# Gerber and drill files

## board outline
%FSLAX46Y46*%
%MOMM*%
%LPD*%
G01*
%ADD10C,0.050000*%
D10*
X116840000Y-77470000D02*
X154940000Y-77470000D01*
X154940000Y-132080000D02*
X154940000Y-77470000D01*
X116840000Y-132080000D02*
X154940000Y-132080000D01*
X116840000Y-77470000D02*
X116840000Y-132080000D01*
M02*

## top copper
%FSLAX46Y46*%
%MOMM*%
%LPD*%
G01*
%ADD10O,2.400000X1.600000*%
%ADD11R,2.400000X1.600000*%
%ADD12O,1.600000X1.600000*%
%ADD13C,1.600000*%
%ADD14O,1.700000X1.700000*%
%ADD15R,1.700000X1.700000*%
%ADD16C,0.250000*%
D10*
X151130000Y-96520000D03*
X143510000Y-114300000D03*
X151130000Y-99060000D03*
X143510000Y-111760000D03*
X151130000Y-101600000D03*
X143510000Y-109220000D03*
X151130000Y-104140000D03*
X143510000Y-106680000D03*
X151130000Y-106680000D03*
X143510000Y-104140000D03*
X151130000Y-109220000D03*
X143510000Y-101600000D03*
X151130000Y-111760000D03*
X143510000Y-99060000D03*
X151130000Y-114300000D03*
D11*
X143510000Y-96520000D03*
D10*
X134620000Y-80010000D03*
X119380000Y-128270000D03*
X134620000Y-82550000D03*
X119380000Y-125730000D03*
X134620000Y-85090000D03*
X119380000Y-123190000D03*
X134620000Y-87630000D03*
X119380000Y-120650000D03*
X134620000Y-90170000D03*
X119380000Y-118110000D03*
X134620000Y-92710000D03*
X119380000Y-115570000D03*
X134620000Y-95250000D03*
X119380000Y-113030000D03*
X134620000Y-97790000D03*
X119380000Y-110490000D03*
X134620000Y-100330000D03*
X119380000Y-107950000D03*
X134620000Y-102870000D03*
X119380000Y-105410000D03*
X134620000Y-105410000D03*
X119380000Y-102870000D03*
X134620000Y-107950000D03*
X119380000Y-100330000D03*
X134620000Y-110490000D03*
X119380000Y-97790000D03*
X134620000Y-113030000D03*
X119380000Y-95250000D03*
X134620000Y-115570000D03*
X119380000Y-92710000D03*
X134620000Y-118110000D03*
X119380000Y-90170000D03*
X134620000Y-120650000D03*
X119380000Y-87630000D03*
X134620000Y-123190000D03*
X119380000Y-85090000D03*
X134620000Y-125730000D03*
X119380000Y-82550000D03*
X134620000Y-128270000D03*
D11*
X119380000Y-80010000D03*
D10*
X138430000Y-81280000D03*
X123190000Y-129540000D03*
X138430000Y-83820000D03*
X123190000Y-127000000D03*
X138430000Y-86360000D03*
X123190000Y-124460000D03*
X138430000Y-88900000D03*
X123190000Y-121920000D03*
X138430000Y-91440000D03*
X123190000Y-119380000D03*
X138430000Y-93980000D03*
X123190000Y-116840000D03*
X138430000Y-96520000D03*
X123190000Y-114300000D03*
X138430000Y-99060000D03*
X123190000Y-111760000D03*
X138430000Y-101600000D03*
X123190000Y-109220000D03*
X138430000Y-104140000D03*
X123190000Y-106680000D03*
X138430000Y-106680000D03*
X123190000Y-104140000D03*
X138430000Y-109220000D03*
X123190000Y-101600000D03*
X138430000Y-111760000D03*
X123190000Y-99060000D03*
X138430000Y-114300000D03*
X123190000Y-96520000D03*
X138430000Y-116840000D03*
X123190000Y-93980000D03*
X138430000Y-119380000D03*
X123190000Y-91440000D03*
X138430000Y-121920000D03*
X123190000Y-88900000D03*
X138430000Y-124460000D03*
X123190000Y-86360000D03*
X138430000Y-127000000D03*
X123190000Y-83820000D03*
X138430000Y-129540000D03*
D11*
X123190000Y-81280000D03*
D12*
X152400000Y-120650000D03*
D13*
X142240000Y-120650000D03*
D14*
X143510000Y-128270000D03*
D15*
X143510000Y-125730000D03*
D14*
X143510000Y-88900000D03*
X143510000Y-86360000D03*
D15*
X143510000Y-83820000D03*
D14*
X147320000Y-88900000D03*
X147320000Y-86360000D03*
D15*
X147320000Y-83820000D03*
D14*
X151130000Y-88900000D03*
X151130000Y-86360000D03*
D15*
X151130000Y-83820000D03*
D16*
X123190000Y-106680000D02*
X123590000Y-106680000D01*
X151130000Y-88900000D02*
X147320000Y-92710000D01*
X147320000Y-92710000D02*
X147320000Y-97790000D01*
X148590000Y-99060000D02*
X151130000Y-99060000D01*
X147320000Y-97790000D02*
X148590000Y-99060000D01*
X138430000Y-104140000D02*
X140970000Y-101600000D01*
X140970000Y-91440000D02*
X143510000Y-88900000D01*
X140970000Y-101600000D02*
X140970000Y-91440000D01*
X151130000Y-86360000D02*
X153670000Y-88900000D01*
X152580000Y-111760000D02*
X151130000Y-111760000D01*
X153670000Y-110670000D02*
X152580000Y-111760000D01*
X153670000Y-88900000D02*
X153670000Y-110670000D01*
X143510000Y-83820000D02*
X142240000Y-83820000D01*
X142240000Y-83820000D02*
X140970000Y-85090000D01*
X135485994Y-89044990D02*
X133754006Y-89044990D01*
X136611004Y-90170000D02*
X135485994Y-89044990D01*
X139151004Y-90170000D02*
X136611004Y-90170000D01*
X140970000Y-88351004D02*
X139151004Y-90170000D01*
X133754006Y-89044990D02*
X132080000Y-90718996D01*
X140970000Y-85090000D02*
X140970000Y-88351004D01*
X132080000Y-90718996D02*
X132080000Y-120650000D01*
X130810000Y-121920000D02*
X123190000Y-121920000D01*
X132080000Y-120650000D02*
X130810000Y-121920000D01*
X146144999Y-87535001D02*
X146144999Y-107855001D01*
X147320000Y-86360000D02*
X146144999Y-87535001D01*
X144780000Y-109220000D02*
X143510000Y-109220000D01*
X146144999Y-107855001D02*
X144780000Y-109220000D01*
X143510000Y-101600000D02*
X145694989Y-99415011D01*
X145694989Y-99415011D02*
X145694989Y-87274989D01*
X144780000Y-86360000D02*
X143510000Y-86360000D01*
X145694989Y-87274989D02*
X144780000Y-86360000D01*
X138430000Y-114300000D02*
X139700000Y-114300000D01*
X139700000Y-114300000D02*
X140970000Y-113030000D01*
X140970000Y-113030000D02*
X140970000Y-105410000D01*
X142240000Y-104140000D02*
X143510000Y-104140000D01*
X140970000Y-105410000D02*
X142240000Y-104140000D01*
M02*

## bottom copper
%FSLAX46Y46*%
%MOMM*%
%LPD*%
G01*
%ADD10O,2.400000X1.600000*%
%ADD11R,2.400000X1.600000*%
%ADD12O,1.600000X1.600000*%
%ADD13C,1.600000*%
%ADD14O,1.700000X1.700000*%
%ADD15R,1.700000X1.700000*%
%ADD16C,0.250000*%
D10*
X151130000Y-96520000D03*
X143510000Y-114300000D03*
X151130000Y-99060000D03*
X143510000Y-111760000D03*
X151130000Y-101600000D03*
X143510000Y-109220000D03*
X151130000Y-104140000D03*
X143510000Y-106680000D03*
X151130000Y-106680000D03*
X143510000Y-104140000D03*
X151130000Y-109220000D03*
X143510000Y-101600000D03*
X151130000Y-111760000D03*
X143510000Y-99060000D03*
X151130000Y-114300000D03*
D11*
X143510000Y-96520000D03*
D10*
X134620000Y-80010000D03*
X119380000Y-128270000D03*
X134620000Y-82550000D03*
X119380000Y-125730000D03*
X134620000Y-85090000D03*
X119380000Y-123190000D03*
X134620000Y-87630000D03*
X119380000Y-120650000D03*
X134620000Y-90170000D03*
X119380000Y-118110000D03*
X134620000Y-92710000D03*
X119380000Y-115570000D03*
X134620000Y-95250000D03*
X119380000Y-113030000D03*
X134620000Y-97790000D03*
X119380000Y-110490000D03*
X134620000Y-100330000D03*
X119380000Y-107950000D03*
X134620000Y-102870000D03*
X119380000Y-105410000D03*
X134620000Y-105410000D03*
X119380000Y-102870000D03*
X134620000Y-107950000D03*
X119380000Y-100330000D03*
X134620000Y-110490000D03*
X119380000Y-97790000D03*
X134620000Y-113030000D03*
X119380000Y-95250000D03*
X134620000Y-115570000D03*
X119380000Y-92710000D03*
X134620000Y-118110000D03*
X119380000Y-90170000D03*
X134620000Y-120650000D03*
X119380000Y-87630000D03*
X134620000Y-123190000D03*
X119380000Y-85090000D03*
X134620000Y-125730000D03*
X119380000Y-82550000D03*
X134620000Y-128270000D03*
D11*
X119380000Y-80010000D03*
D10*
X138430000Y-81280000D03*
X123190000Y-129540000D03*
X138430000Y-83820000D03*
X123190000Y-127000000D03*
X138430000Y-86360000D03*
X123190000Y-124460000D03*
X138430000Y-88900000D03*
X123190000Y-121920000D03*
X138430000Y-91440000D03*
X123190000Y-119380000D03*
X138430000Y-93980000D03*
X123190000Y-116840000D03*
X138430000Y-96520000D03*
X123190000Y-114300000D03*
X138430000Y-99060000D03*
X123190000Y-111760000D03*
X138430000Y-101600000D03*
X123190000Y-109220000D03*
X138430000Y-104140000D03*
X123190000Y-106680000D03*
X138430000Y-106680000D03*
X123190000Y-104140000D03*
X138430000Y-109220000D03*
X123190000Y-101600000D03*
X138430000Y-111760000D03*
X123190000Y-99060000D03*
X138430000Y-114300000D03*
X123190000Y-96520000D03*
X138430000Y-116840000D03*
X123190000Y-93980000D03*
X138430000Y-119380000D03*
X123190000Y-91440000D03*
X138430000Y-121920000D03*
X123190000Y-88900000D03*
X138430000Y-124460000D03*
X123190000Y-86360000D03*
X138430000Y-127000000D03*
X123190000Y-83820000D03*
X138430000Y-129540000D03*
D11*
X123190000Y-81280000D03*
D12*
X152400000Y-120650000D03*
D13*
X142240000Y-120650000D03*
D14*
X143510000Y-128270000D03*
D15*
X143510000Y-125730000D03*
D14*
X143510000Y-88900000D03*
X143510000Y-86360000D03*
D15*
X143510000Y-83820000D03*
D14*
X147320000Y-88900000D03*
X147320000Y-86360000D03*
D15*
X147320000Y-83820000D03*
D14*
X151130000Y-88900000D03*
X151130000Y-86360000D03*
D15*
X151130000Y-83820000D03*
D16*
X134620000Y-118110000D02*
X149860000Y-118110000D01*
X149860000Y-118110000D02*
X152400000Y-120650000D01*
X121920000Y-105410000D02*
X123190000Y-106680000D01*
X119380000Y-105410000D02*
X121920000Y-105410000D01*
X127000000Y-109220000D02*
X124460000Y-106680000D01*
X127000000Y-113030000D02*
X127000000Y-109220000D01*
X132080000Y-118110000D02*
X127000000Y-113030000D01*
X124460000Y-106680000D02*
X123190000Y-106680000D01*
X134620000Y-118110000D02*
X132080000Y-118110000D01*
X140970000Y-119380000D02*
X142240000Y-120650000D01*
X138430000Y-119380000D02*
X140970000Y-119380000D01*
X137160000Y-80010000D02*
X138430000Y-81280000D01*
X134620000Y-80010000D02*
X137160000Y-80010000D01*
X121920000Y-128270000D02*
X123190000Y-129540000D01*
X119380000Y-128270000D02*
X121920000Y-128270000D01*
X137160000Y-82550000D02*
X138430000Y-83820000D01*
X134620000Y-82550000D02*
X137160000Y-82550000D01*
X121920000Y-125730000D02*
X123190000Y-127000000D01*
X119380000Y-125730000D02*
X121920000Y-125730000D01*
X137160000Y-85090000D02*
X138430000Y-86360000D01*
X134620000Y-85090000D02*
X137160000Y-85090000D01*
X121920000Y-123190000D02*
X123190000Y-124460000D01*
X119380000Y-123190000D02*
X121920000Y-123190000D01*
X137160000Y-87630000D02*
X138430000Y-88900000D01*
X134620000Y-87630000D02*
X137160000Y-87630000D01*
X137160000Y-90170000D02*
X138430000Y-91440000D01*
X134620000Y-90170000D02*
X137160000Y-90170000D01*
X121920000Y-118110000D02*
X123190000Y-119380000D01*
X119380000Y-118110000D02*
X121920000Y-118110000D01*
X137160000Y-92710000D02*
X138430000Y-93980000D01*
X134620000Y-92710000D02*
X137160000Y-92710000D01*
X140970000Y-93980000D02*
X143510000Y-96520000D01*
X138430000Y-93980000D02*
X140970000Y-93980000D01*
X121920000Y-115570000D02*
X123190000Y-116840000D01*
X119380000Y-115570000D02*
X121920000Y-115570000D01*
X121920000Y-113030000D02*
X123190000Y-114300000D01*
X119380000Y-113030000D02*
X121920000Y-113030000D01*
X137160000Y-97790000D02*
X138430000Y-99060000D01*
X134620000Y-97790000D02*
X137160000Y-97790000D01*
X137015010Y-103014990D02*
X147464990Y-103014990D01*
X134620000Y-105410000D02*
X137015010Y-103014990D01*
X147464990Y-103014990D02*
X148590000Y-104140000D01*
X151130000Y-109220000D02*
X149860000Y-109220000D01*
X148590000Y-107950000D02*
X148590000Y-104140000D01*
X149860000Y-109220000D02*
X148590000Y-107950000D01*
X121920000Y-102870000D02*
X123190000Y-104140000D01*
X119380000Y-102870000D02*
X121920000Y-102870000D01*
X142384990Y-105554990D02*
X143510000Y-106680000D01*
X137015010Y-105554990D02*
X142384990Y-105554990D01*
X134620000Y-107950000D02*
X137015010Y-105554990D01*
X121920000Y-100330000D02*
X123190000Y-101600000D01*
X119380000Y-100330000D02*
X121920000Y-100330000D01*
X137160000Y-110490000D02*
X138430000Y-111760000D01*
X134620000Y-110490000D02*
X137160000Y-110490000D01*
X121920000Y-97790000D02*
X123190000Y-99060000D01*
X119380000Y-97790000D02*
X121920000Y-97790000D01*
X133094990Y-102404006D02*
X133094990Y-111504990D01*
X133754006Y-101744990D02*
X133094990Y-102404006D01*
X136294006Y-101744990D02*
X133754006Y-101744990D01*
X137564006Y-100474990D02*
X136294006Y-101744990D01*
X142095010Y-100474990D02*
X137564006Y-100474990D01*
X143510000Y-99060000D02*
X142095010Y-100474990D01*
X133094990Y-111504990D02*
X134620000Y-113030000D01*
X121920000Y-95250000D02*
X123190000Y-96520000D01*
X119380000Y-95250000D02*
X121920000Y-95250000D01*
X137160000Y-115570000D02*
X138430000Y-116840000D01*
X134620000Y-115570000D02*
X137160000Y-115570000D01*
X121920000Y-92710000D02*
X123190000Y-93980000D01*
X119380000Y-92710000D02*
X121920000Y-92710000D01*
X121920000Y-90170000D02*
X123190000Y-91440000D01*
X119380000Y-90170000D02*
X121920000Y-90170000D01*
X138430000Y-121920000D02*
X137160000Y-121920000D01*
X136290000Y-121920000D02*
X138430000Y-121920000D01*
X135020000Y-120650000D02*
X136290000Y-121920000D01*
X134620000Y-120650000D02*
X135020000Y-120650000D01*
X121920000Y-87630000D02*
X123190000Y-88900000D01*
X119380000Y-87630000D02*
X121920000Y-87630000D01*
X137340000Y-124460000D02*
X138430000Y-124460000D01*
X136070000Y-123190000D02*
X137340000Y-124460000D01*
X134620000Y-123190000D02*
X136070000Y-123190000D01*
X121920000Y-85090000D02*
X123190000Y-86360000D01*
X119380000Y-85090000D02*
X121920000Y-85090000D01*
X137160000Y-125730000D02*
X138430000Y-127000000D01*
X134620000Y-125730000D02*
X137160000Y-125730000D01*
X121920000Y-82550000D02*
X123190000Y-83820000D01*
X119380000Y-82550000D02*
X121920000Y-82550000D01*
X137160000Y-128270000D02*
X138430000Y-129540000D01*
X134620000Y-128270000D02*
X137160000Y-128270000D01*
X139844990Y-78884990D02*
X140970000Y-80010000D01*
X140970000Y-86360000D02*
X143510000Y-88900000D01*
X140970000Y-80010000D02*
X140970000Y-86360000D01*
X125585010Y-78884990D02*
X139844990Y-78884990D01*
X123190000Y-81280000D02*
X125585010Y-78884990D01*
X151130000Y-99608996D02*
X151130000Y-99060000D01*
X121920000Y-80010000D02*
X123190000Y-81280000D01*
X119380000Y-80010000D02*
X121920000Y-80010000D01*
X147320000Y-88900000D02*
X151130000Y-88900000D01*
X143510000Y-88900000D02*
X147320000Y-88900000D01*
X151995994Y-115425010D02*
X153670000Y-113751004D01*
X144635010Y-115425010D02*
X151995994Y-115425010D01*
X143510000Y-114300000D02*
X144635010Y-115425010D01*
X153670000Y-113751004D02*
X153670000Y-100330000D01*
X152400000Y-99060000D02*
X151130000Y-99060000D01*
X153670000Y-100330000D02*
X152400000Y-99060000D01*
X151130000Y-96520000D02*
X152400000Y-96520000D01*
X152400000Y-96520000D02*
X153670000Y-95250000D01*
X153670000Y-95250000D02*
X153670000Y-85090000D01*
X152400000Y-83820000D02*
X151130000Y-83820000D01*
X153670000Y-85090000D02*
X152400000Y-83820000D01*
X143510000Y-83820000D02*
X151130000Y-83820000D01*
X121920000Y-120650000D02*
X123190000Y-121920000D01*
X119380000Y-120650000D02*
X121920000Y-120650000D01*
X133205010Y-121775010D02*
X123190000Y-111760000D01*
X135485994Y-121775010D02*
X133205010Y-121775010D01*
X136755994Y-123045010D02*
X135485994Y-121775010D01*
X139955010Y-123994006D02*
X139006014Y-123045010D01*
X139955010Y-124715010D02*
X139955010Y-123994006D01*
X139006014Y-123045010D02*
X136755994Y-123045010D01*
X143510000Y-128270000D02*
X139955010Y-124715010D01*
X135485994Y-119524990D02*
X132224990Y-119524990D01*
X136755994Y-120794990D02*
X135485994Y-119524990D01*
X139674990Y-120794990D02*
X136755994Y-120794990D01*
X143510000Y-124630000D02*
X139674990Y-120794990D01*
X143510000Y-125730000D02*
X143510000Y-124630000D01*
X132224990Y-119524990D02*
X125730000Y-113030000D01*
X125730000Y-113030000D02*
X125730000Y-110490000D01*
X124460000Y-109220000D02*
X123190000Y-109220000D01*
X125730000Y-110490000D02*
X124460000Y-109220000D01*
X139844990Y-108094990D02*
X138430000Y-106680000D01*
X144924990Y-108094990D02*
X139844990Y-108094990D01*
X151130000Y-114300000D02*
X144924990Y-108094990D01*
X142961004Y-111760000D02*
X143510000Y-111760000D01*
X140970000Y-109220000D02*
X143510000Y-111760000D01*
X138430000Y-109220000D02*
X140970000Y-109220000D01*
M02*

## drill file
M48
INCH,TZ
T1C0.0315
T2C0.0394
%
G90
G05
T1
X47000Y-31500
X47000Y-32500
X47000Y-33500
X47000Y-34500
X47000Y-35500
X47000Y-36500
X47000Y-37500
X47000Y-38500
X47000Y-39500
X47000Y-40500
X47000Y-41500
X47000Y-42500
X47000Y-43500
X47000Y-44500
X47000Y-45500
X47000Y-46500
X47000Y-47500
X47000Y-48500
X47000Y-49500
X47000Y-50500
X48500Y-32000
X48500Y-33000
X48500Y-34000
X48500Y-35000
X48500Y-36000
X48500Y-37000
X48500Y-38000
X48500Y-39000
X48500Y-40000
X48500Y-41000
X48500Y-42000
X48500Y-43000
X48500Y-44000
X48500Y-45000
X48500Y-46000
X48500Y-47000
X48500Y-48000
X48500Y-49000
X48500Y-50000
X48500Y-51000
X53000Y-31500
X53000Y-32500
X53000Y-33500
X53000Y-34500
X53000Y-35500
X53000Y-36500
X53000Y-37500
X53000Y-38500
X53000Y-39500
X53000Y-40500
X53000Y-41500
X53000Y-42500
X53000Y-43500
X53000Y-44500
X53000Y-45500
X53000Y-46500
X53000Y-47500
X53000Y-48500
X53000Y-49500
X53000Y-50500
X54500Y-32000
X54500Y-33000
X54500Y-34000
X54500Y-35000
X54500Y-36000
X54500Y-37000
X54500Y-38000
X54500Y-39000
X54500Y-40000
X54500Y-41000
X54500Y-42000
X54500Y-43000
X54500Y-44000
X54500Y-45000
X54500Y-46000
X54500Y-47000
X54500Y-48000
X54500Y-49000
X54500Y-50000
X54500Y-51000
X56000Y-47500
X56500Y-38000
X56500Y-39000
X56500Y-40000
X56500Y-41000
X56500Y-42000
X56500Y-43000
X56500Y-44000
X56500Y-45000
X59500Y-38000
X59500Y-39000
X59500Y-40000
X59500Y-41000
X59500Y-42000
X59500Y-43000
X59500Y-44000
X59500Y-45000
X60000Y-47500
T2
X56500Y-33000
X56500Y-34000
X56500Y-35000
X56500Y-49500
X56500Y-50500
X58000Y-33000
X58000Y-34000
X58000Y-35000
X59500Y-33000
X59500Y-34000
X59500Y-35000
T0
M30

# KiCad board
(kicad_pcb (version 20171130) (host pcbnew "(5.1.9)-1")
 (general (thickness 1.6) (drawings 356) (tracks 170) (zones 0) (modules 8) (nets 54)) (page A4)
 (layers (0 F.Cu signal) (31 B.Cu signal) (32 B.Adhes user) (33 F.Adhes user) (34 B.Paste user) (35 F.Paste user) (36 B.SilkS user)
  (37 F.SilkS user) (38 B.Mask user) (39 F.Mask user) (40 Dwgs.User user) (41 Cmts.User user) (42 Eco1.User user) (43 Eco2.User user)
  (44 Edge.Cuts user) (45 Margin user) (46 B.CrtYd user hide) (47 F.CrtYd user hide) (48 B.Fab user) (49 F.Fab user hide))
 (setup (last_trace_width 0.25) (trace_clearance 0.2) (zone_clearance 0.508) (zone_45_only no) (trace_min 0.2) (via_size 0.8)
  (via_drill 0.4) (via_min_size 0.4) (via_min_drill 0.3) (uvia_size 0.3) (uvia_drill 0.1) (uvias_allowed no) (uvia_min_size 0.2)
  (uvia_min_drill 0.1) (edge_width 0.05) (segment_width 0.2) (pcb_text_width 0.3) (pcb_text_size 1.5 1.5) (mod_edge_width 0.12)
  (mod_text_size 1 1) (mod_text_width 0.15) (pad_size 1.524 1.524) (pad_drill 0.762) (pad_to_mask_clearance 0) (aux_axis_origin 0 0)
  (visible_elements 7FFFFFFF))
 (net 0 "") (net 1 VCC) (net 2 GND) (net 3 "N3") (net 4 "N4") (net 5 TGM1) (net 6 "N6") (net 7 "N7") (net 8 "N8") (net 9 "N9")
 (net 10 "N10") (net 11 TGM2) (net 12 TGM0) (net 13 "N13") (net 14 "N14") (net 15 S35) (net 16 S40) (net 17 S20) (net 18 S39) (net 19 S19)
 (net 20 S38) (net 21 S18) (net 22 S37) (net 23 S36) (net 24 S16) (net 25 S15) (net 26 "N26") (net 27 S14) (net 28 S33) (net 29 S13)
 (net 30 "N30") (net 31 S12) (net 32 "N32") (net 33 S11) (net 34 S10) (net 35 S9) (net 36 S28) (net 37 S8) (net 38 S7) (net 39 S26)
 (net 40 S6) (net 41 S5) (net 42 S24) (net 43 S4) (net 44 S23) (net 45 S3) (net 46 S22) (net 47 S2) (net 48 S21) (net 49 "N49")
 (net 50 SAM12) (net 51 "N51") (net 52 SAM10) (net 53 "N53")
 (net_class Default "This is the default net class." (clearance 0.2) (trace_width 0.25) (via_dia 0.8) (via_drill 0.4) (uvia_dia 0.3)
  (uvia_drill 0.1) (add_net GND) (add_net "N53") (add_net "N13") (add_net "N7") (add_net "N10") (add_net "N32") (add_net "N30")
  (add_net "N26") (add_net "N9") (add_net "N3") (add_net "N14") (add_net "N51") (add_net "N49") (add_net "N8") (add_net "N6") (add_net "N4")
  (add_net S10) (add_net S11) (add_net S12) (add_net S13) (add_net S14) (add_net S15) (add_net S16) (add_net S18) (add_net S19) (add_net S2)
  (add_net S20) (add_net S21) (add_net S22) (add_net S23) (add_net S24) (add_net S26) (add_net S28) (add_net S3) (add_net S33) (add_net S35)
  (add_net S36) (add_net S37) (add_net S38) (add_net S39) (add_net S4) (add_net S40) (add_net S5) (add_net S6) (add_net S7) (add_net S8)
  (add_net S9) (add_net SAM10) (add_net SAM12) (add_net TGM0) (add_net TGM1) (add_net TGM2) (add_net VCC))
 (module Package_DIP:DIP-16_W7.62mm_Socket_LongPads (layer F.Cu) (at 143.51 96.52)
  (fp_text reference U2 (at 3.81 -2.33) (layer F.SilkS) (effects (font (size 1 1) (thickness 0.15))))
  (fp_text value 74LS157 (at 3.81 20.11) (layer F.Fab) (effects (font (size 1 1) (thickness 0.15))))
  (pad 16 thru_hole oval (at 7.62 0) (size 2.4 1.6) (drill 0.8) (layers *.Cu *.Mask) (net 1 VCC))
  (pad 8 thru_hole oval (at 0 17.78) (size 2.4 1.6) (drill 0.8) (layers *.Cu *.Mask) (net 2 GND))
  (pad 15 thru_hole oval (at 7.62 2.54) (size 2.4 1.6) (drill 0.8) (layers *.Cu *.Mask) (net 2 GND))
  (pad 7 thru_hole oval (at 0 15.24) (size 2.4 1.6) (drill 0.8) (layers *.Cu *.Mask) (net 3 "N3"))
  (pad 14 thru_hole oval (at 7.62 5.08) (size 2.4 1.6) (drill 0.8) (layers *.Cu *.Mask) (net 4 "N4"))
  (pad 6 thru_hole oval (at 0 12.7) (size 2.4 1.6) (drill 0.8) (layers *.Cu *.Mask) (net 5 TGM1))
  (pad 13 thru_hole oval (at 7.62 7.62) (size 2.4 1.6) (drill 0.8) (layers *.Cu *.Mask) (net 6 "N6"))
  (pad 5 thru_hole oval (at 0 10.16) (size 2.4 1.6) (drill 0.8) (layers *.Cu *.Mask) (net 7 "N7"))
  (pad 12 thru_hole oval (at 7.62 10.16) (size 2.4 1.6) (drill 0.8) (layers *.Cu *.Mask) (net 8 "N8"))
  (pad 4 thru_hole oval (at 0 7.62) (size 2.4 1.6) (drill 0.8) (layers *.Cu *.Mask) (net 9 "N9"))
  (pad 11 thru_hole oval (at 7.62 12.7) (size 2.4 1.6) (drill 0.8) (layers *.Cu *.Mask) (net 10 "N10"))
  (pad 3 thru_hole oval (at 0 5.08) (size 2.4 1.6) (drill 0.8) (layers *.Cu *.Mask) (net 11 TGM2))
  (pad 10 thru_hole oval (at 7.62 15.24) (size 2.4 1.6) (drill 0.8) (layers *.Cu *.Mask) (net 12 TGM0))
  (pad 2 thru_hole oval (at 0 2.54) (size 2.4 1.6) (drill 0.8) (layers *.Cu *.Mask) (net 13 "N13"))
  (pad 9 thru_hole oval (at 7.62 17.78) (size 2.4 1.6) (drill 0.8) (layers *.Cu *.Mask) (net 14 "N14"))
  (pad 1 thru_hole rect (at 0 0) (size 2.4 1.6) (drill 0.8) (layers *.Cu *.Mask) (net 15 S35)))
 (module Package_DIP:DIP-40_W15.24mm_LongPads (layer F.Cu) (at 119.38 80.01)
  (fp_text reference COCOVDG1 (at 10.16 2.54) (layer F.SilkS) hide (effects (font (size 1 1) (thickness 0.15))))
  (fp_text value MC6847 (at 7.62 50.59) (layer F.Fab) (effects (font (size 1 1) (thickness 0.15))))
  (pad 40 thru_hole oval (at 15.24 0) (size 2.4 1.6) (drill 0.8) (layers *.Cu *.Mask) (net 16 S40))
  (pad 20 thru_hole oval (at 0 48.26) (size 2.4 1.6) (drill 0.8) (layers *.Cu *.Mask) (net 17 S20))
  (pad 39 thru_hole oval (at 15.24 2.54) (size 2.4 1.6) (drill 0.8) (layers *.Cu *.Mask) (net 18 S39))
  (pad 19 thru_hole oval (at 0 45.72) (size 2.4 1.6) (drill 0.8) (layers *.Cu *.Mask) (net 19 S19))
  (pad 38 thru_hole oval (at 15.24 5.08) (size 2.4 1.6) (drill 0.8) (layers *.Cu *.Mask) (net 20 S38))
  (pad 18 thru_hole oval (at 0 43.18) (size 2.4 1.6) (drill 0.8) (layers *.Cu *.Mask) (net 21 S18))
  (pad 37 thru_hole oval (at 15.24 7.62) (size 2.4 1.6) (drill 0.8) (layers *.Cu *.Mask) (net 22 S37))
  (pad 17 thru_hole oval (at 0 40.64) (size 2.4 1.6) (drill 0.8) (layers *.Cu *.Mask) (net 1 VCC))
  (pad 36 thru_hole oval (at 15.24 10.16) (size 2.4 1.6) (drill 0.8) (layers *.Cu *.Mask) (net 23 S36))
  (pad 16 thru_hole oval (at 0 38.1) (size 2.4 1.6) (drill 0.8) (layers *.Cu *.Mask) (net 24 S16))
  (pad 35 thru_hole oval (at 15.24 12.7) (size 2.4 1.6) (drill 0.8) (layers *.Cu *.Mask) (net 15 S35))
  (pad 15 thru_hole oval (at 0 35.56) (size 2.4 1.6) (drill 0.8) (layers *.Cu *.Mask) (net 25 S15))
  (pad 34 thru_hole oval (at 15.24 15.24) (size 2.4 1.6) (drill 0.8) (layers *.Cu *.Mask) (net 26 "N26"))
  (pad 14 thru_hole oval (at 0 33.02) (size 2.4 1.6) (drill 0.8) (layers *.Cu *.Mask) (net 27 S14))
  (pad 33 thru_hole oval (at 15.24 17.78) (size 2.4 1.6) (drill 0.8) (layers *.Cu *.Mask) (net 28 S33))
  (pad 13 thru_hole oval (at 0 30.48) (size 2.4 1.6) (drill 0.8) (layers *.Cu *.Mask) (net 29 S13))
  (pad 32 thru_hole oval (at 15.24 20.32) (size 2.4 1.6) (drill 0.8) (layers *.Cu *.Mask) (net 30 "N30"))
  (pad 12 thru_hole oval (at 0 27.94) (size 2.4 1.6) (drill 0.8) (layers *.Cu *.Mask) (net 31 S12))
  (pad 31 thru_hole oval (at 15.24 22.86) (size 2.4 1.6) (drill 0.8) (layers *.Cu *.Mask) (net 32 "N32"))
  (pad 11 thru_hole oval (at 0 25.4) (size 2.4 1.6) (drill 0.8) (layers *.Cu *.Mask) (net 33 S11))
  (pad 30 thru_hole oval (at 15.24 25.4) (size 2.4 1.6) (drill 0.8) (layers *.Cu *.Mask) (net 10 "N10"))
  (pad 10 thru_hole oval (at 0 22.86) (size 2.4 1.6) (drill 0.8) (layers *.Cu *.Mask) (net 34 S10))
  (pad 29 thru_hole oval (at 15.24 27.94) (size 2.4 1.6) (drill 0.8) (layers *.Cu *.Mask) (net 7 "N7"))
  (pad 9 thru_hole oval (at 0 20.32) (size 2.4 1.6) (drill 0.8) (layers *.Cu *.Mask) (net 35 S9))
  (pad 28 thru_hole oval (at 15.24 30.48) (size 2.4 1.6) (drill 0.8) (layers *.Cu *.Mask) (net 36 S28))
  (pad 8 thru_hole oval (at 0 17.78) (size 2.4 1.6) (drill 0.8) (layers *.Cu *.Mask) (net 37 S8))
  (pad 27 thru_hole oval (at 15.24 33.02) (size 2.4 1.6) (drill 0.8) (layers *.Cu *.Mask) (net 13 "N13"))
  (pad 7 thru_hole oval (at 0 15.24) (size 2.4 1.6) (drill 0.8) (layers *.Cu *.Mask) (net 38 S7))
  (pad 26 thru_hole oval (at 15.24 35.56) (size 2.4 1.6) (drill 0.8) (layers *.Cu *.Mask) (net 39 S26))
  (pad 6 thru_hole oval (at 0 12.7) (size 2.4 1.6) (drill 0.8) (layers *.Cu *.Mask) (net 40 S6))
  (pad 25 thru_hole oval (at 15.24 38.1) (size 2.4 1.6) (drill 0.8) (layers *.Cu *.Mask) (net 33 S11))
  (pad 5 thru_hole oval (at 0 10.16) (size 2.4 1.6) (drill 0.8) (layers *.Cu *.Mask) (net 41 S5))
  (pad 24 thru_hole oval (at 15.24 40.64) (size 2.4 1.6) (drill 0.8) (layers *.Cu *.Mask) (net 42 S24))
  (pad 4 thru_hole oval (at 0 7.62) (size 2.4 1.6) (drill 0.8) (layers *.Cu *.Mask) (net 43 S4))
  (pad 23 thru_hole oval (at 15.24 43.18) (size 2.4 1.6) (drill 0.8) (layers *.Cu *.Mask) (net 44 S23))
  (pad 3 thru_hole oval (at 0 5.08) (size 2.4 1.6) (drill 0.8) (layers *.Cu *.Mask) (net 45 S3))
  (pad 22 thru_hole oval (at 15.24 45.72) (size 2.4 1.6) (drill 0.8) (layers *.Cu *.Mask) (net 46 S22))
  (pad 2 thru_hole oval (at 0 2.54) (size 2.4 1.6) (drill 0.8) (layers *.Cu *.Mask) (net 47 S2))
  (pad 21 thru_hole oval (at 15.24 48.26) (size 2.4 1.6) (drill 0.8) (layers *.Cu *.Mask) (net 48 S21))
  (pad 1 thru_hole rect (at 0 0) (size 2.4 1.6) (drill 0.8) (layers *.Cu *.Mask) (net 2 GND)))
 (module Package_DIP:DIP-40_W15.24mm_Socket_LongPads (layer F.Cu) (at 123.19 81.28)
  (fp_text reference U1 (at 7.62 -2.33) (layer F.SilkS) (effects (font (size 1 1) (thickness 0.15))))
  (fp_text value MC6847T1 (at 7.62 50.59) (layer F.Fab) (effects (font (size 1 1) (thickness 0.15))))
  (pad 40 thru_hole oval (at 15.24 0) (size 2.4 1.6) (drill 0.8) (layers *.Cu *.Mask) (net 16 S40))
  (pad 20 thru_hole oval (at 0 48.26) (size 2.4 1.6) (drill 0.8) (layers *.Cu *.Mask) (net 17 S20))
  (pad 39 thru_hole oval (at 15.24 2.54) (size 2.4 1.6) (drill 0.8) (layers *.Cu *.Mask) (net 18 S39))
  (pad 19 thru_hole oval (at 0 45.72) (size 2.4 1.6) (drill 0.8) (layers *.Cu *.Mask) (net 19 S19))
  (pad 38 thru_hole oval (at 15.24 5.08) (size 2.4 1.6) (drill 0.8) (layers *.Cu *.Mask) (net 20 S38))
  (pad 18 thru_hole oval (at 0 43.18) (size 2.4 1.6) (drill 0.8) (layers *.Cu *.Mask) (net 21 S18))
  (pad 37 thru_hole oval (at 15.24 7.62) (size 2.4 1.6) (drill 0.8) (layers *.Cu *.Mask) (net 22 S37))
  (pad 17 thru_hole oval (at 0 40.64) (size 2.4 1.6) (drill 0.8) (layers *.Cu *.Mask) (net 1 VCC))
  (pad 36 thru_hole oval (at 15.24 10.16) (size 2.4 1.6) (drill 0.8) (layers *.Cu *.Mask) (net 23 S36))
  (pad 16 thru_hole oval (at 0 38.1) (size 2.4 1.6) (drill 0.8) (layers *.Cu *.Mask) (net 24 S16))
  (pad 35 thru_hole oval (at 15.24 12.7) (size 2.4 1.6) (drill 0.8) (layers *.Cu *.Mask) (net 15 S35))
  (pad 15 thru_hole oval (at 0 35.56) (size 2.4 1.6) (drill 0.8) (layers *.Cu *.Mask) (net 25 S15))
  (pad 34 thru_hole oval (at 15.24 15.24) (size 2.4 1.6) (drill 0.8) (layers *.Cu *.Mask) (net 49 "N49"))
  (pad 14 thru_hole oval (at 0 33.02) (size 2.4 1.6) (drill 0.8) (layers *.Cu *.Mask) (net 27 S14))
  (pad 33 thru_hole oval (at 15.24 17.78) (size 2.4 1.6) (drill 0.8) (layers *.Cu *.Mask) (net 28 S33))
  (pad 13 thru_hole oval (at 0 30.48) (size 2.4 1.6) (drill 0.8) (layers *.Cu *.Mask) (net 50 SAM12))
  (pad 32 thru_hole oval (at 15.24 20.32) (size 2.4 1.6) (drill 0.8) (layers *.Cu *.Mask) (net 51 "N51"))
  (pad 12 thru_hole oval (at 0 27.94) (size 2.4 1.6) (drill 0.8) (layers *.Cu *.Mask) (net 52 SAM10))
  (pad 31 thru_hole oval (at 15.24 22.86) (size 2.4 1.6) (drill 0.8) (layers *.Cu *.Mask) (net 2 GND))
  (pad 11 thru_hole oval (at 0 25.4) (size 2.4 1.6) (drill 0.8) (layers *.Cu *.Mask) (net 33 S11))
  (pad 30 thru_hole oval (at 15.24 25.4) (size 2.4 1.6) (drill 0.8) (layers *.Cu *.Mask) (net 14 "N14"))
  (pad 10 thru_hole oval (at 0 22.86) (size 2.4 1.6) (drill 0.8) (layers *.Cu *.Mask) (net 34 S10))
  (pad 29 thru_hole oval (at 15.24 27.94) (size 2.4 1.6) (drill 0.8) (layers *.Cu *.Mask) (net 3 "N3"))
  (pad 9 thru_hole oval (at 0 20.32) (size 2.4 1.6) (drill 0.8) (layers *.Cu *.Mask) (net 35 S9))
  (pad 28 thru_hole oval (at 15.24 30.48) (size 2.4 1.6) (drill 0.8) (layers *.Cu *.Mask) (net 36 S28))
  (pad 8 thru_hole oval (at 0 17.78) (size 2.4 1.6) (drill 0.8) (layers *.Cu *.Mask) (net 37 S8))
  (pad 27 thru_hole oval (at 15.24 33.02) (size 2.4 1.6) (drill 0.8) (layers *.Cu *.Mask) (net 9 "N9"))
  (pad 7 thru_hole oval (at 0 15.24) (size 2.4 1.6) (drill 0.8) (layers *.Cu *.Mask) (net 38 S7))
  (pad 26 thru_hole oval (at 15.24 35.56) (size 2.4 1.6) (drill 0.8) (layers *.Cu *.Mask) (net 39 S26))
  (pad 6 thru_hole oval (at 0 12.7) (size 2.4 1.6) (drill 0.8) (layers *.Cu *.Mask) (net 40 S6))
  (pad 25 thru_hole oval (at 15.24 38.1) (size 2.4 1.6) (drill 0.8) (layers *.Cu *.Mask) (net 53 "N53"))
  (pad 5 thru_hole oval (at 0 10.16) (size 2.4 1.6) (drill 0.8) (layers *.Cu *.Mask) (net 41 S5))
  (pad 24 thru_hole oval (at 15.24 40.64) (size 2.4 1.6) (drill 0.8) (layers *.Cu *.Mask) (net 42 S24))
  (pad 4 thru_hole oval (at 0 7.62) (size 2.4 1.6) (drill 0.8) (layers *.Cu *.Mask) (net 43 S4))
  (pad 23 thru_hole oval (at 15.24 43.18) (size 2.4 1.6) (drill 0.8) (layers *.Cu *.Mask) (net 44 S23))
  (pad 3 thru_hole oval (at 0 5.08) (size 2.4 1.6) (drill 0.8) (layers *.Cu *.Mask) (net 45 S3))
  (pad 22 thru_hole oval (at 15.24 45.72) (size 2.4 1.6) (drill 0.8) (layers *.Cu *.Mask) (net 46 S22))
  (pad 2 thru_hole oval (at 0 2.54) (size 2.4 1.6) (drill 0.8) (layers *.Cu *.Mask) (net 47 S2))
  (pad 21 thru_hole oval (at 15.24 48.26) (size 2.4 1.6) (drill 0.8) (layers *.Cu *.Mask) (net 48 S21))
  (pad 1 thru_hole rect (at 0 0) (size 2.4 1.6) (drill 0.8) (layers *.Cu *.Mask) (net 2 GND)))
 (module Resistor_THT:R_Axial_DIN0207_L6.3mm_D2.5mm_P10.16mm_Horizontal (layer F.Cu) (at 142.24 120.65)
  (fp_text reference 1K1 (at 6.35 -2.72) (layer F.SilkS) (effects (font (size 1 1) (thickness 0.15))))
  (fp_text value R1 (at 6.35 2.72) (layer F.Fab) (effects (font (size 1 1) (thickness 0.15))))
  (pad 2 thru_hole oval (at 10.16 0) (size 1.6 1.6) (drill 0.8) (layers *.Cu *.Mask) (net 33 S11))
  (pad 1 thru_hole circle (at 0 0) (size 1.6 1.6) (drill 0.8) (layers *.Cu *.Mask) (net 53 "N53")))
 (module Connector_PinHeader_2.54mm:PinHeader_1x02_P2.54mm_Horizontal (layer F.Cu) (at 143.51 125.73)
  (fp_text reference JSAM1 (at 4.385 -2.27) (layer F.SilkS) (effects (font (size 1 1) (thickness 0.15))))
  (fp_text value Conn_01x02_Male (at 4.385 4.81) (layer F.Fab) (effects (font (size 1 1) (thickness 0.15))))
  (pad 2 thru_hole oval (at 0 2.54) (size 1.7 1.7) (drill 1) (layers *.Cu *.Mask) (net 50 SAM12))
  (pad 1 thru_hole rect (at 0 0) (size 1.7 1.7) (drill 1) (layers *.Cu *.Mask) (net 52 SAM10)))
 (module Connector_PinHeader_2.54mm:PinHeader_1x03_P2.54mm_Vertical (layer F.Cu) (at 143.51 83.82)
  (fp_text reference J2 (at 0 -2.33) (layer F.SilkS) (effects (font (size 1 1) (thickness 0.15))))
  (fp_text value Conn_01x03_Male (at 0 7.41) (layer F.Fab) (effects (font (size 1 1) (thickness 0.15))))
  (pad 3 thru_hole oval (at 0 5.08) (size 1.7 1.7) (drill 1) (layers *.Cu *.Mask) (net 2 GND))
  (pad 2 thru_hole oval (at 0 2.54) (size 1.7 1.7) (drill 1) (layers *.Cu *.Mask) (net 11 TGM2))
  (pad 1 thru_hole rect (at 0 0) (size 1.7 1.7) (drill 1) (layers *.Cu *.Mask) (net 1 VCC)))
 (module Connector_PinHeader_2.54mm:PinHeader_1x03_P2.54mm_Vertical (layer F.Cu) (at 147.32 83.82)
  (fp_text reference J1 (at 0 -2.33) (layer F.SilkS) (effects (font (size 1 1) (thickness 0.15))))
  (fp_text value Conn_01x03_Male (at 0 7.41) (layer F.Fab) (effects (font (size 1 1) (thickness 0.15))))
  (pad 3 thru_hole oval (at 0 5.08) (size 1.7 1.7) (drill 1) (layers *.Cu *.Mask) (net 2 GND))
  (pad 2 thru_hole oval (at 0 2.54) (size 1.7 1.7) (drill 1) (layers *.Cu *.Mask) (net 5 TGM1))
  (pad 1 thru_hole rect (at 0 0) (size 1.7 1.7) (drill 1) (layers *.Cu *.Mask) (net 1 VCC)))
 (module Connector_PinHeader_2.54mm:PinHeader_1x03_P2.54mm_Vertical (layer F.Cu) (at 151.13 83.82)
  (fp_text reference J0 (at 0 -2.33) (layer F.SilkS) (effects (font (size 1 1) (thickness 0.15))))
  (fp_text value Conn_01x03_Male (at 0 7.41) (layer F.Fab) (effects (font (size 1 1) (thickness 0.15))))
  (pad 3 thru_hole oval (at 0 5.08) (size 1.7 1.7) (drill 1) (layers *.Cu *.Mask) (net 2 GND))
  (pad 2 thru_hole oval (at 0 2.54) (size 1.7 1.7) (drill 1) (layers *.Cu *.Mask) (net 12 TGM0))
  (pad 1 thru_hole rect (at 0 0) (size 1.7 1.7) (drill 1) (layers *.Cu *.Mask) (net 1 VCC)))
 (gr_line (start 116.84 77.47) (end 154.94 77.47) (layer Edge.Cuts) (width 0.05))
 (gr_line (start 154.94 132.08) (end 154.94 77.47) (layer Edge.Cuts) (width 0.05))
 (gr_line (start 116.84 132.08) (end 154.94 132.08) (layer Edge.Cuts) (width 0.05))
 (gr_line (start 116.84 77.47) (end 116.84 132.08) (layer Edge.Cuts) (width 0.05))
 (segment (start 123.19 106.68) (end 123.59 106.68) (width 0.25) (layer F.Cu) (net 33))
 (segment (start 134.62 118.11) (end 149.86 118.11) (width 0.25) (layer B.Cu) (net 33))
 (segment (start 149.86 118.11) (end 152.4 120.65) (width 0.25) (layer B.Cu) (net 33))
 (segment (start 121.92 105.41) (end 123.19 106.68) (width 0.25) (layer B.Cu) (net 33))
 (segment (start 119.38 105.41) (end 121.92 105.41) (width 0.25) (layer B.Cu) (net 33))
 (segment (start 127 109.22) (end 124.46 106.68) (width 0.25) (layer B.Cu) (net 33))
 (segment (start 127 113.03) (end 127 109.22) (width 0.25) (layer B.Cu) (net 33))
 (segment (start 132.08 118.11) (end 127 113.03) (width 0.25) (layer B.Cu) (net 33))
 (segment (start 124.46 106.68) (end 123.19 106.68) (width 0.25) (layer B.Cu) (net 33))
 (segment (start 134.62 118.11) (end 132.08 118.11) (width 0.25) (layer B.Cu) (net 33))
 (segment (start 140.97 119.38) (end 142.24 120.65) (width 0.25) (layer B.Cu) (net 53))
 (segment (start 138.43 119.38) (end 140.97 119.38) (width 0.25) (layer B.Cu) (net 53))
 (segment (start 137.16 80.01) (end 138.43 81.28) (width 0.25) (layer B.Cu) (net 16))
 (segment (start 134.62 80.01) (end 137.16 80.01) (width 0.25) (layer B.Cu) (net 16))
 (segment (start 121.92 128.27) (end 123.19 129.54) (width 0.25) (layer B.Cu) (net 17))
 (segment (start 119.38 128.27) (end 121.92 128.27) (width 0.25) (layer B.Cu) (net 17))
 (segment (start 137.16 82.55) (end 138.43 83.82) (width 0.25) (layer B.Cu) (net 18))
 (segment (start 134.62 82.55) (end 137.16 82.55) (width 0.25) (layer B.Cu) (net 18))
 (segment (start 121.92 125.73) (end 123.19 127) (width 0.25) (layer B.Cu) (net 19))
 (segment (start 119.38 125.73) (end 121.92 125.73) (width 0.25) (layer B.Cu) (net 19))
 (segment (start 137.16 85.09) (end 138.43 86.36) (width 0.25) (layer B.Cu) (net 20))
 (segment (start 134.62 85.09) (end 137.16 85.09) (width 0.25) (layer B.Cu) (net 20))
 (segment (start 121.92 123.19) (end 123.19 124.46) (width 0.25) (layer B.Cu) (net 21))
 (segment (start 119.38 123.19) (end 121.92 123.19) (width 0.25) (layer B.Cu) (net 21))
 (segment (start 137.16 87.63) (end 138.43 88.9) (width 0.25) (layer B.Cu) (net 22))
 (segment (start 134.62 87.63) (end 137.16 87.63) (width 0.25) (layer B.Cu) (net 22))
 (segment (start 137.16 90.17) (end 138.43 91.44) (width 0.25) (layer B.Cu) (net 23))
 (segment (start 134.62 90.17) (end 137.16 90.17) (width 0.25) (layer B.Cu) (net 23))
 (segment (start 121.92 118.11) (end 123.19 119.38) (width 0.25) (layer B.Cu) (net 24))
 (segment (start 119.38 118.11) (end 121.92 118.11) (width 0.25) (layer B.Cu) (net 24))
 (segment (start 137.16 92.71) (end 138.43 93.98) (width 0.25) (layer B.Cu) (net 15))
 (segment (start 134.62 92.71) (end 137.16 92.71) (width 0.25) (layer B.Cu) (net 15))
 (segment (start 140.97 93.98) (end 143.51 96.52) (width 0.25) (layer B.Cu) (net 15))
 (segment (start 138.43 93.98) (end 140.97 93.98) (width 0.25) (layer B.Cu) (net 15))
 (segment (start 121.92 115.57) (end 123.19 116.84) (width 0.25) (layer B.Cu) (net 25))
 (segment (start 119.38 115.57) (end 121.92 115.57) (width 0.25) (layer B.Cu) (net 25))
 (segment (start 121.92 113.03) (end 123.19 114.3) (width 0.25) (layer B.Cu) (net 27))
 (segment (start 119.38 113.03) (end 121.92 113.03) (width 0.25) (layer B.Cu) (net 27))
 (segment (start 137.16 97.79) (end 138.43 99.06) (width 0.25) (layer B.Cu) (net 28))
 (segment (start 134.62 97.79) (end 137.16 97.79) (width 0.25) (layer B.Cu) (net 28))
 (segment (start 137.01501 103.01499) (end 147.46499 103.01499) (width 0.25) (layer B.Cu) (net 10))
 (segment (start 134.62 105.41) (end 137.01501 103.01499) (width 0.25) (layer B.Cu) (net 10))
 (segment (start 147.46499 103.01499) (end 148.59 104.14) (width 0.25) (layer B.Cu) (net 10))
 (segment (start 151.13 109.22) (end 149.86 109.22) (width 0.25) (layer B.Cu) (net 10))
 (segment (start 148.59 107.95) (end 148.59 104.14) (width 0.25) (layer B.Cu) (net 10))
 (segment (start 149.86 109.22) (end 148.59 107.95) (width 0.25) (layer B.Cu) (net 10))
 (segment (start 121.92 102.87) (end 123.19 104.14) (width 0.25) (layer B.Cu) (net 34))
 (segment (start 119.38 102.87) (end 121.92 102.87) (width 0.25) (layer B.Cu) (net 34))
 (segment (start 142.38499 105.55499) (end 143.51 106.68) (width 0.25) (layer B.Cu) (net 7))
 (segment (start 137.01501 105.55499) (end 142.38499 105.55499) (width 0.25) (layer B.Cu) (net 7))
 (segment (start 134.62 107.95) (end 137.01501 105.55499) (width 0.25) (layer B.Cu) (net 7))
 (segment (start 121.92 100.33) (end 123.19 101.6) (width 0.25) (layer B.Cu) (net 35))
 (segment (start 119.38 100.33) (end 121.92 100.33) (width 0.25) (layer B.Cu) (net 35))
 (segment (start 137.16 110.49) (end 138.43 111.76) (width 0.25) (layer B.Cu) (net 36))
 (segment (start 134.62 110.49) (end 137.16 110.49) (width 0.25) (layer B.Cu) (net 36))
 (segment (start 121.92 97.79) (end 123.19 99.06) (width 0.25) (layer B.Cu) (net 37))
 (segment (start 119.38 97.79) (end 121.92 97.79) (width 0.25) (layer B.Cu) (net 37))
 (segment (start 133.09499 102.404006) (end 133.09499 111.50499) (width 0.25) (layer B.Cu) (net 13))
 (segment (start 133.754006 101.74499) (end 133.09499 102.404006) (width 0.25) (layer B.Cu) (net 13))
 (segment (start 136.294006 101.74499) (end 133.754006 101.74499) (width 0.25) (layer B.Cu) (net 13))
 (segment (start 137.564006 100.47499) (end 136.294006 101.74499) (width 0.25) (layer B.Cu) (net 13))
 (segment (start 142.09501 100.47499) (end 137.564006 100.47499) (width 0.25) (layer B.Cu) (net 13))
 (segment (start 143.51 99.06) (end 142.09501 100.47499) (width 0.25) (layer B.Cu) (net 13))
 (segment (start 133.09499 111.50499) (end 134.62 113.03) (width 0.25) (layer B.Cu) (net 13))
 (segment (start 121.92 95.25) (end 123.19 96.52) (width 0.25) (layer B.Cu) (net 38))
 (segment (start 119.38 95.25) (end 121.92 95.25) (width 0.25) (layer B.Cu) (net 38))
 (segment (start 137.16 115.57) (end 138.43 116.84) (width 0.25) (layer B.Cu) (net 39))
 (segment (start 134.62 115.57) (end 137.16 115.57) (width 0.25) (layer B.Cu) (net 39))
 (segment (start 121.92 92.71) (end 123.19 93.98) (width 0.25) (layer B.Cu) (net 40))
 (segment (start 119.38 92.71) (end 121.92 92.71) (width 0.25) (layer B.Cu) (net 40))
 (segment (start 121.92 90.17) (end 123.19 91.44) (width 0.25) (layer B.Cu) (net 41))
 (segment (start 119.38 90.17) (end 121.92 90.17) (width 0.25) (layer B.Cu) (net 41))
 (segment (start 138.43 121.92) (end 137.16 121.92) (width 0.25) (layer B.Cu) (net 42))
 (segment (start 136.29 121.92) (end 138.43 121.92) (width 0.25) (layer B.Cu) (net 42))
 (segment (start 135.02 120.65) (end 136.29 121.92) (width 0.25) (layer B.Cu) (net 42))
 (segment (start 134.62 120.65) (end 135.02 120.65) (width 0.25) (layer B.Cu) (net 42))
 (segment (start 121.92 87.63) (end 123.19 88.9) (width 0.25) (layer B.Cu) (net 43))
 (segment (start 119.38 87.63) (end 121.92 87.63) (width 0.25) (layer B.Cu) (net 43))
 (segment (start 137.34 124.46) (end 138.43 124.46) (width 0.25) (layer B.Cu) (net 44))
 (segment (start 136.07 123.19) (end 137.34 124.46) (width 0.25) (layer B.Cu) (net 44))
 (segment (start 134.62 123.19) (end 136.07 123.19) (width 0.25) (layer B.Cu) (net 44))
 (segment (start 121.92 85.09) (end 123.19 86.36) (width 0.25) (layer B.Cu) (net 45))
 (segment (start 119.38 85.09) (end 121.92 85.09) (width 0.25) (layer B.Cu) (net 45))
 (segment (start 137.16 125.73) (end 138.43 127) (width 0.25) (layer B.Cu) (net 46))
 (segment (start 134.62 125.73) (end 137.16 125.73) (width 0.25) (layer B.Cu) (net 46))
 (segment (start 121.92 82.55) (end 123.19 83.82) (width 0.25) (layer B.Cu) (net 47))
 (segment (start 119.38 82.55) (end 121.92 82.55) (width 0.25) (layer B.Cu) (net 47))
 (segment (start 137.16 128.27) (end 138.43 129.54) (width 0.25) (layer B.Cu) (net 48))
 (segment (start 134.62 128.27) (end 137.16 128.27) (width 0.25) (layer B.Cu) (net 48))
 (segment (start 139.84499 78.88499) (end 140.97 80.01) (width 0.25) (layer B.Cu) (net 2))
 (segment (start 140.97 86.36) (end 143.51 88.9) (width 0.25) (layer B.Cu) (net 2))
 (segment (start 140.97 80.01) (end 140.97 86.36) (width 0.25) (layer B.Cu) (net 2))
 (segment (start 151.13 88.9) (end 147.32 92.71) (width 0.25) (layer F.Cu) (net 2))
 (segment (start 147.32 92.71) (end 147.32 97.79) (width 0.25) (layer F.Cu) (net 2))
 (segment (start 148.59 99.06) (end 151.13 99.06) (width 0.25) (layer F.Cu) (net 2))
 (segment (start 147.32 97.79) (end 148.59 99.06) (width 0.25) (layer F.Cu) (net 2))
 (segment (start 125.58501 78.88499) (end 139.84499 78.88499) (width 0.25) (layer B.Cu) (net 2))
 (segment (start 123.19 81.28) (end 125.58501 78.88499) (width 0.25) (layer B.Cu) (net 2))
 (segment (start 151.13 99.608996) (end 151.13 99.06) (width 0.25) (layer B.Cu) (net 2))
 (segment (start 121.92 80.01) (end 123.19 81.28) (width 0.25) (layer B.Cu) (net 2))
 (segment (start 119.38 80.01) (end 121.92 80.01) (width 0.25) (layer B.Cu) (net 2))
 (segment (start 147.32 88.9) (end 151.13 88.9) (width 0.25) (layer B.Cu) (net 2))
 (segment (start 143.51 88.9) (end 147.32 88.9) (width 0.25) (layer B.Cu) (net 2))
 (segment (start 138.43 104.14) (end 140.97 101.6) (width 0.25) (layer F.Cu) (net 2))
 (segment (start 140.97 91.44) (end 143.51 88.9) (width 0.25) (layer F.Cu) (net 2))
 (segment (start 140.97 101.6) (end 140.97 91.44) (width 0.25) (layer F.Cu) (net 2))
 (segment (start 151.995994 115.42501) (end 153.67 113.751004) (width 0.25) (layer B.Cu) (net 2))
 (segment (start 144.63501 115.42501) (end 151.995994 115.42501) (width 0.25) (layer B.Cu) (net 2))
 (segment (start 143.51 114.3) (end 144.63501 115.42501) (width 0.25) (layer B.Cu) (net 2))
 (segment (start 153.67 113.751004) (end 153.67 100.33) (width 0.25) (layer B.Cu) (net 2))
 (segment (start 152.4 99.06) (end 151.13 99.06) (width 0.25) (layer B.Cu) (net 2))
 (segment (start 153.67 100.33) (end 152.4 99.06) (width 0.25) (layer B.Cu) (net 2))
 (segment (start 151.13 86.36) (end 153.67 88.9) (width 0.25) (layer F.Cu) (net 12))
 (segment (start 152.58 111.76) (end 151.13 111.76) (width 0.25) (layer F.Cu) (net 12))
 (segment (start 153.67 110.67) (end 152.58 111.76) (width 0.25) (layer F.Cu) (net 12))
 (segment (start 153.67 88.9) (end 153.67 110.67) (width 0.25) (layer F.Cu) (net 12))
 (segment (start 151.13 96.52) (end 152.4 96.52) (width 0.25) (layer B.Cu) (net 1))
 (segment (start 152.4 96.52) (end 153.67 95.25) (width 0.25) (layer B.Cu) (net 1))
 (segment (start 153.67 95.25) (end 153.67 85.09) (width 0.25) (layer B.Cu) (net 1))
 (segment (start 152.4 83.82) (end 151.13 83.82) (width 0.25) (layer B.Cu) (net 1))
 (segment (start 153.67 85.09) (end 152.4 83.82) (width 0.25) (layer B.Cu) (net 1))
 (segment (start 143.51 83.82) (end 151.13 83.82) (width 0.25) (layer B.Cu) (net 1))
 (segment (start 121.92 120.65) (end 123.19 121.92) (width 0.25) (layer B.Cu) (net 1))
 (segment (start 119.38 120.65) (end 121.92 120.65) (width 0.25) (layer B.Cu) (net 1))
 (segment (start 143.51 83.82) (end 142.24 83.82) (width 0.25) (layer F.Cu) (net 1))
 (segment (start 142.24 83.82) (end 140.97 85.09) (width 0.25) (layer F.Cu) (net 1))
 (segment (start 135.485994 89.04499) (end 133.754006 89.04499) (width 0.25) (layer F.Cu) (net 1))
 (segment (start 136.611004 90.17) (end 135.485994 89.04499) (width 0.25) (layer F.Cu) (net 1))
 (segment (start 139.151004 90.17) (end 136.611004 90.17) (width 0.25) (layer F.Cu) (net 1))
 (segment (start 140.97 88.351004) (end 139.151004 90.17) (width 0.25) (layer F.Cu) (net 1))
 (segment (start 133.754006 89.04499) (end 132.08 90.718996) (width 0.25) (layer F.Cu) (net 1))
 (segment (start 140.97 85.09) (end 140.97 88.351004) (width 0.25) (layer F.Cu) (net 1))
 (segment (start 132.08 90.718996) (end 132.08 120.65) (width 0.25) (layer F.Cu) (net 1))
 (segment (start 130.81 121.92) (end 123.19 121.92) (width 0.25) (layer F.Cu) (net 1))
 (segment (start 132.08 120.65) (end 130.81 121.92) (width 0.25) (layer F.Cu) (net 1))
 (segment (start 146.144999 87.535001) (end 146.144999 107.855001) (width 0.25) (layer F.Cu) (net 5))
 (segment (start 147.32 86.36) (end 146.144999 87.535001) (width 0.25) (layer F.Cu) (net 5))
 (segment (start 144.78 109.22) (end 143.51 109.22) (width 0.25) (layer F.Cu) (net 5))
 (segment (start 146.144999 107.855001) (end 144.78 109.22) (width 0.25) (layer F.Cu) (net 5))
 (segment (start 143.51 101.6) (end 145.694989 99.415011) (width 0.25) (layer F.Cu) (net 11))
 (segment (start 145.694989 99.415011) (end 145.694989 87.274989) (width 0.25) (layer F.Cu) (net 11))
 (segment (start 144.78 86.36) (end 143.51 86.36) (width 0.25) (layer F.Cu) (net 11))
 (segment (start 145.694989 87.274989) (end 144.78 86.36) (width 0.25) (layer F.Cu) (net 11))
 (segment (start 133.20501 121.77501) (end 123.19 111.76) (width 0.25) (layer B.Cu) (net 50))
 (segment (start 135.485994 121.77501) (end 133.20501 121.77501) (width 0.25) (layer B.Cu) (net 50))
 (segment (start 136.755994 123.04501) (end 135.485994 121.77501) (width 0.25) (layer B.Cu) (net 50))
 (segment (start 139.95501 123.994006) (end 139.006014 123.04501) (width 0.25) (layer B.Cu) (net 50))
 (segment (start 139.95501 124.71501) (end 139.95501 123.994006) (width 0.25) (layer B.Cu) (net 50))
 (segment (start 139.006014 123.04501) (end 136.755994 123.04501) (width 0.25) (layer B.Cu) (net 50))
 (segment (start 143.51 128.27) (end 139.95501 124.71501) (width 0.25) (layer B.Cu) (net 50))
 (segment (start 135.485994 119.52499) (end 132.22499 119.52499) (width 0.25) (layer B.Cu) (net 52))
 (segment (start 136.755994 120.79499) (end 135.485994 119.52499) (width 0.25) (layer B.Cu) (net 52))
 (segment (start 139.67499 120.79499) (end 136.755994 120.79499) (width 0.25) (layer B.Cu) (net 52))
 (segment (start 143.51 124.63) (end 139.67499 120.79499) (width 0.25) (layer B.Cu) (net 52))
 (segment (start 143.51 125.73) (end 143.51 124.63) (width 0.25) (layer B.Cu) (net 52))
 (segment (start 132.22499 119.52499) (end 125.73 113.03) (width 0.25) (layer B.Cu) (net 52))
 (segment (start 125.73 113.03) (end 125.73 110.49) (width 0.25) (layer B.Cu) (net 52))
 (segment (start 124.46 109.22) (end 123.19 109.22) (width 0.25) (layer B.Cu) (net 52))
 (segment (start 125.73 110.49) (end 124.46 109.22) (width 0.25) (layer B.Cu) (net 52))
 (segment (start 139.84499 108.09499) (end 138.43 106.68) (width 0.25) (layer B.Cu) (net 14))
 (segment (start 144.92499 108.09499) (end 139.84499 108.09499) (width 0.25) (layer B.Cu) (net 14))
 (segment (start 151.13 114.3) (end 144.92499 108.09499) (width 0.25) (layer B.Cu) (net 14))
 (segment (start 142.961004 111.76) (end 143.51 111.76) (width 0.25) (layer B.Cu) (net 3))
 (segment (start 140.97 109.22) (end 143.51 111.76) (width 0.25) (layer B.Cu) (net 3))
 (segment (start 138.43 109.22) (end 140.97 109.22) (width 0.25) (layer B.Cu) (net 3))
 (segment (start 138.43 114.3) (end 139.7 114.3) (width 0.25) (layer F.Cu) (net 9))
 (segment (start 139.7 114.3) (end 140.97 113.03) (width 0.25) (layer F.Cu) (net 9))
 (segment (start 140.97 113.03) (end 140.97 105.41) (width 0.25) (layer F.Cu) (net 9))
 (segment (start 142.24 104.14) (end 143.51 104.14) (width 0.25) (layer F.Cu) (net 9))
 (segment (start 140.97 105.41) (end 142.24 104.14) (width 0.25) (layer F.Cu) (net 9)))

